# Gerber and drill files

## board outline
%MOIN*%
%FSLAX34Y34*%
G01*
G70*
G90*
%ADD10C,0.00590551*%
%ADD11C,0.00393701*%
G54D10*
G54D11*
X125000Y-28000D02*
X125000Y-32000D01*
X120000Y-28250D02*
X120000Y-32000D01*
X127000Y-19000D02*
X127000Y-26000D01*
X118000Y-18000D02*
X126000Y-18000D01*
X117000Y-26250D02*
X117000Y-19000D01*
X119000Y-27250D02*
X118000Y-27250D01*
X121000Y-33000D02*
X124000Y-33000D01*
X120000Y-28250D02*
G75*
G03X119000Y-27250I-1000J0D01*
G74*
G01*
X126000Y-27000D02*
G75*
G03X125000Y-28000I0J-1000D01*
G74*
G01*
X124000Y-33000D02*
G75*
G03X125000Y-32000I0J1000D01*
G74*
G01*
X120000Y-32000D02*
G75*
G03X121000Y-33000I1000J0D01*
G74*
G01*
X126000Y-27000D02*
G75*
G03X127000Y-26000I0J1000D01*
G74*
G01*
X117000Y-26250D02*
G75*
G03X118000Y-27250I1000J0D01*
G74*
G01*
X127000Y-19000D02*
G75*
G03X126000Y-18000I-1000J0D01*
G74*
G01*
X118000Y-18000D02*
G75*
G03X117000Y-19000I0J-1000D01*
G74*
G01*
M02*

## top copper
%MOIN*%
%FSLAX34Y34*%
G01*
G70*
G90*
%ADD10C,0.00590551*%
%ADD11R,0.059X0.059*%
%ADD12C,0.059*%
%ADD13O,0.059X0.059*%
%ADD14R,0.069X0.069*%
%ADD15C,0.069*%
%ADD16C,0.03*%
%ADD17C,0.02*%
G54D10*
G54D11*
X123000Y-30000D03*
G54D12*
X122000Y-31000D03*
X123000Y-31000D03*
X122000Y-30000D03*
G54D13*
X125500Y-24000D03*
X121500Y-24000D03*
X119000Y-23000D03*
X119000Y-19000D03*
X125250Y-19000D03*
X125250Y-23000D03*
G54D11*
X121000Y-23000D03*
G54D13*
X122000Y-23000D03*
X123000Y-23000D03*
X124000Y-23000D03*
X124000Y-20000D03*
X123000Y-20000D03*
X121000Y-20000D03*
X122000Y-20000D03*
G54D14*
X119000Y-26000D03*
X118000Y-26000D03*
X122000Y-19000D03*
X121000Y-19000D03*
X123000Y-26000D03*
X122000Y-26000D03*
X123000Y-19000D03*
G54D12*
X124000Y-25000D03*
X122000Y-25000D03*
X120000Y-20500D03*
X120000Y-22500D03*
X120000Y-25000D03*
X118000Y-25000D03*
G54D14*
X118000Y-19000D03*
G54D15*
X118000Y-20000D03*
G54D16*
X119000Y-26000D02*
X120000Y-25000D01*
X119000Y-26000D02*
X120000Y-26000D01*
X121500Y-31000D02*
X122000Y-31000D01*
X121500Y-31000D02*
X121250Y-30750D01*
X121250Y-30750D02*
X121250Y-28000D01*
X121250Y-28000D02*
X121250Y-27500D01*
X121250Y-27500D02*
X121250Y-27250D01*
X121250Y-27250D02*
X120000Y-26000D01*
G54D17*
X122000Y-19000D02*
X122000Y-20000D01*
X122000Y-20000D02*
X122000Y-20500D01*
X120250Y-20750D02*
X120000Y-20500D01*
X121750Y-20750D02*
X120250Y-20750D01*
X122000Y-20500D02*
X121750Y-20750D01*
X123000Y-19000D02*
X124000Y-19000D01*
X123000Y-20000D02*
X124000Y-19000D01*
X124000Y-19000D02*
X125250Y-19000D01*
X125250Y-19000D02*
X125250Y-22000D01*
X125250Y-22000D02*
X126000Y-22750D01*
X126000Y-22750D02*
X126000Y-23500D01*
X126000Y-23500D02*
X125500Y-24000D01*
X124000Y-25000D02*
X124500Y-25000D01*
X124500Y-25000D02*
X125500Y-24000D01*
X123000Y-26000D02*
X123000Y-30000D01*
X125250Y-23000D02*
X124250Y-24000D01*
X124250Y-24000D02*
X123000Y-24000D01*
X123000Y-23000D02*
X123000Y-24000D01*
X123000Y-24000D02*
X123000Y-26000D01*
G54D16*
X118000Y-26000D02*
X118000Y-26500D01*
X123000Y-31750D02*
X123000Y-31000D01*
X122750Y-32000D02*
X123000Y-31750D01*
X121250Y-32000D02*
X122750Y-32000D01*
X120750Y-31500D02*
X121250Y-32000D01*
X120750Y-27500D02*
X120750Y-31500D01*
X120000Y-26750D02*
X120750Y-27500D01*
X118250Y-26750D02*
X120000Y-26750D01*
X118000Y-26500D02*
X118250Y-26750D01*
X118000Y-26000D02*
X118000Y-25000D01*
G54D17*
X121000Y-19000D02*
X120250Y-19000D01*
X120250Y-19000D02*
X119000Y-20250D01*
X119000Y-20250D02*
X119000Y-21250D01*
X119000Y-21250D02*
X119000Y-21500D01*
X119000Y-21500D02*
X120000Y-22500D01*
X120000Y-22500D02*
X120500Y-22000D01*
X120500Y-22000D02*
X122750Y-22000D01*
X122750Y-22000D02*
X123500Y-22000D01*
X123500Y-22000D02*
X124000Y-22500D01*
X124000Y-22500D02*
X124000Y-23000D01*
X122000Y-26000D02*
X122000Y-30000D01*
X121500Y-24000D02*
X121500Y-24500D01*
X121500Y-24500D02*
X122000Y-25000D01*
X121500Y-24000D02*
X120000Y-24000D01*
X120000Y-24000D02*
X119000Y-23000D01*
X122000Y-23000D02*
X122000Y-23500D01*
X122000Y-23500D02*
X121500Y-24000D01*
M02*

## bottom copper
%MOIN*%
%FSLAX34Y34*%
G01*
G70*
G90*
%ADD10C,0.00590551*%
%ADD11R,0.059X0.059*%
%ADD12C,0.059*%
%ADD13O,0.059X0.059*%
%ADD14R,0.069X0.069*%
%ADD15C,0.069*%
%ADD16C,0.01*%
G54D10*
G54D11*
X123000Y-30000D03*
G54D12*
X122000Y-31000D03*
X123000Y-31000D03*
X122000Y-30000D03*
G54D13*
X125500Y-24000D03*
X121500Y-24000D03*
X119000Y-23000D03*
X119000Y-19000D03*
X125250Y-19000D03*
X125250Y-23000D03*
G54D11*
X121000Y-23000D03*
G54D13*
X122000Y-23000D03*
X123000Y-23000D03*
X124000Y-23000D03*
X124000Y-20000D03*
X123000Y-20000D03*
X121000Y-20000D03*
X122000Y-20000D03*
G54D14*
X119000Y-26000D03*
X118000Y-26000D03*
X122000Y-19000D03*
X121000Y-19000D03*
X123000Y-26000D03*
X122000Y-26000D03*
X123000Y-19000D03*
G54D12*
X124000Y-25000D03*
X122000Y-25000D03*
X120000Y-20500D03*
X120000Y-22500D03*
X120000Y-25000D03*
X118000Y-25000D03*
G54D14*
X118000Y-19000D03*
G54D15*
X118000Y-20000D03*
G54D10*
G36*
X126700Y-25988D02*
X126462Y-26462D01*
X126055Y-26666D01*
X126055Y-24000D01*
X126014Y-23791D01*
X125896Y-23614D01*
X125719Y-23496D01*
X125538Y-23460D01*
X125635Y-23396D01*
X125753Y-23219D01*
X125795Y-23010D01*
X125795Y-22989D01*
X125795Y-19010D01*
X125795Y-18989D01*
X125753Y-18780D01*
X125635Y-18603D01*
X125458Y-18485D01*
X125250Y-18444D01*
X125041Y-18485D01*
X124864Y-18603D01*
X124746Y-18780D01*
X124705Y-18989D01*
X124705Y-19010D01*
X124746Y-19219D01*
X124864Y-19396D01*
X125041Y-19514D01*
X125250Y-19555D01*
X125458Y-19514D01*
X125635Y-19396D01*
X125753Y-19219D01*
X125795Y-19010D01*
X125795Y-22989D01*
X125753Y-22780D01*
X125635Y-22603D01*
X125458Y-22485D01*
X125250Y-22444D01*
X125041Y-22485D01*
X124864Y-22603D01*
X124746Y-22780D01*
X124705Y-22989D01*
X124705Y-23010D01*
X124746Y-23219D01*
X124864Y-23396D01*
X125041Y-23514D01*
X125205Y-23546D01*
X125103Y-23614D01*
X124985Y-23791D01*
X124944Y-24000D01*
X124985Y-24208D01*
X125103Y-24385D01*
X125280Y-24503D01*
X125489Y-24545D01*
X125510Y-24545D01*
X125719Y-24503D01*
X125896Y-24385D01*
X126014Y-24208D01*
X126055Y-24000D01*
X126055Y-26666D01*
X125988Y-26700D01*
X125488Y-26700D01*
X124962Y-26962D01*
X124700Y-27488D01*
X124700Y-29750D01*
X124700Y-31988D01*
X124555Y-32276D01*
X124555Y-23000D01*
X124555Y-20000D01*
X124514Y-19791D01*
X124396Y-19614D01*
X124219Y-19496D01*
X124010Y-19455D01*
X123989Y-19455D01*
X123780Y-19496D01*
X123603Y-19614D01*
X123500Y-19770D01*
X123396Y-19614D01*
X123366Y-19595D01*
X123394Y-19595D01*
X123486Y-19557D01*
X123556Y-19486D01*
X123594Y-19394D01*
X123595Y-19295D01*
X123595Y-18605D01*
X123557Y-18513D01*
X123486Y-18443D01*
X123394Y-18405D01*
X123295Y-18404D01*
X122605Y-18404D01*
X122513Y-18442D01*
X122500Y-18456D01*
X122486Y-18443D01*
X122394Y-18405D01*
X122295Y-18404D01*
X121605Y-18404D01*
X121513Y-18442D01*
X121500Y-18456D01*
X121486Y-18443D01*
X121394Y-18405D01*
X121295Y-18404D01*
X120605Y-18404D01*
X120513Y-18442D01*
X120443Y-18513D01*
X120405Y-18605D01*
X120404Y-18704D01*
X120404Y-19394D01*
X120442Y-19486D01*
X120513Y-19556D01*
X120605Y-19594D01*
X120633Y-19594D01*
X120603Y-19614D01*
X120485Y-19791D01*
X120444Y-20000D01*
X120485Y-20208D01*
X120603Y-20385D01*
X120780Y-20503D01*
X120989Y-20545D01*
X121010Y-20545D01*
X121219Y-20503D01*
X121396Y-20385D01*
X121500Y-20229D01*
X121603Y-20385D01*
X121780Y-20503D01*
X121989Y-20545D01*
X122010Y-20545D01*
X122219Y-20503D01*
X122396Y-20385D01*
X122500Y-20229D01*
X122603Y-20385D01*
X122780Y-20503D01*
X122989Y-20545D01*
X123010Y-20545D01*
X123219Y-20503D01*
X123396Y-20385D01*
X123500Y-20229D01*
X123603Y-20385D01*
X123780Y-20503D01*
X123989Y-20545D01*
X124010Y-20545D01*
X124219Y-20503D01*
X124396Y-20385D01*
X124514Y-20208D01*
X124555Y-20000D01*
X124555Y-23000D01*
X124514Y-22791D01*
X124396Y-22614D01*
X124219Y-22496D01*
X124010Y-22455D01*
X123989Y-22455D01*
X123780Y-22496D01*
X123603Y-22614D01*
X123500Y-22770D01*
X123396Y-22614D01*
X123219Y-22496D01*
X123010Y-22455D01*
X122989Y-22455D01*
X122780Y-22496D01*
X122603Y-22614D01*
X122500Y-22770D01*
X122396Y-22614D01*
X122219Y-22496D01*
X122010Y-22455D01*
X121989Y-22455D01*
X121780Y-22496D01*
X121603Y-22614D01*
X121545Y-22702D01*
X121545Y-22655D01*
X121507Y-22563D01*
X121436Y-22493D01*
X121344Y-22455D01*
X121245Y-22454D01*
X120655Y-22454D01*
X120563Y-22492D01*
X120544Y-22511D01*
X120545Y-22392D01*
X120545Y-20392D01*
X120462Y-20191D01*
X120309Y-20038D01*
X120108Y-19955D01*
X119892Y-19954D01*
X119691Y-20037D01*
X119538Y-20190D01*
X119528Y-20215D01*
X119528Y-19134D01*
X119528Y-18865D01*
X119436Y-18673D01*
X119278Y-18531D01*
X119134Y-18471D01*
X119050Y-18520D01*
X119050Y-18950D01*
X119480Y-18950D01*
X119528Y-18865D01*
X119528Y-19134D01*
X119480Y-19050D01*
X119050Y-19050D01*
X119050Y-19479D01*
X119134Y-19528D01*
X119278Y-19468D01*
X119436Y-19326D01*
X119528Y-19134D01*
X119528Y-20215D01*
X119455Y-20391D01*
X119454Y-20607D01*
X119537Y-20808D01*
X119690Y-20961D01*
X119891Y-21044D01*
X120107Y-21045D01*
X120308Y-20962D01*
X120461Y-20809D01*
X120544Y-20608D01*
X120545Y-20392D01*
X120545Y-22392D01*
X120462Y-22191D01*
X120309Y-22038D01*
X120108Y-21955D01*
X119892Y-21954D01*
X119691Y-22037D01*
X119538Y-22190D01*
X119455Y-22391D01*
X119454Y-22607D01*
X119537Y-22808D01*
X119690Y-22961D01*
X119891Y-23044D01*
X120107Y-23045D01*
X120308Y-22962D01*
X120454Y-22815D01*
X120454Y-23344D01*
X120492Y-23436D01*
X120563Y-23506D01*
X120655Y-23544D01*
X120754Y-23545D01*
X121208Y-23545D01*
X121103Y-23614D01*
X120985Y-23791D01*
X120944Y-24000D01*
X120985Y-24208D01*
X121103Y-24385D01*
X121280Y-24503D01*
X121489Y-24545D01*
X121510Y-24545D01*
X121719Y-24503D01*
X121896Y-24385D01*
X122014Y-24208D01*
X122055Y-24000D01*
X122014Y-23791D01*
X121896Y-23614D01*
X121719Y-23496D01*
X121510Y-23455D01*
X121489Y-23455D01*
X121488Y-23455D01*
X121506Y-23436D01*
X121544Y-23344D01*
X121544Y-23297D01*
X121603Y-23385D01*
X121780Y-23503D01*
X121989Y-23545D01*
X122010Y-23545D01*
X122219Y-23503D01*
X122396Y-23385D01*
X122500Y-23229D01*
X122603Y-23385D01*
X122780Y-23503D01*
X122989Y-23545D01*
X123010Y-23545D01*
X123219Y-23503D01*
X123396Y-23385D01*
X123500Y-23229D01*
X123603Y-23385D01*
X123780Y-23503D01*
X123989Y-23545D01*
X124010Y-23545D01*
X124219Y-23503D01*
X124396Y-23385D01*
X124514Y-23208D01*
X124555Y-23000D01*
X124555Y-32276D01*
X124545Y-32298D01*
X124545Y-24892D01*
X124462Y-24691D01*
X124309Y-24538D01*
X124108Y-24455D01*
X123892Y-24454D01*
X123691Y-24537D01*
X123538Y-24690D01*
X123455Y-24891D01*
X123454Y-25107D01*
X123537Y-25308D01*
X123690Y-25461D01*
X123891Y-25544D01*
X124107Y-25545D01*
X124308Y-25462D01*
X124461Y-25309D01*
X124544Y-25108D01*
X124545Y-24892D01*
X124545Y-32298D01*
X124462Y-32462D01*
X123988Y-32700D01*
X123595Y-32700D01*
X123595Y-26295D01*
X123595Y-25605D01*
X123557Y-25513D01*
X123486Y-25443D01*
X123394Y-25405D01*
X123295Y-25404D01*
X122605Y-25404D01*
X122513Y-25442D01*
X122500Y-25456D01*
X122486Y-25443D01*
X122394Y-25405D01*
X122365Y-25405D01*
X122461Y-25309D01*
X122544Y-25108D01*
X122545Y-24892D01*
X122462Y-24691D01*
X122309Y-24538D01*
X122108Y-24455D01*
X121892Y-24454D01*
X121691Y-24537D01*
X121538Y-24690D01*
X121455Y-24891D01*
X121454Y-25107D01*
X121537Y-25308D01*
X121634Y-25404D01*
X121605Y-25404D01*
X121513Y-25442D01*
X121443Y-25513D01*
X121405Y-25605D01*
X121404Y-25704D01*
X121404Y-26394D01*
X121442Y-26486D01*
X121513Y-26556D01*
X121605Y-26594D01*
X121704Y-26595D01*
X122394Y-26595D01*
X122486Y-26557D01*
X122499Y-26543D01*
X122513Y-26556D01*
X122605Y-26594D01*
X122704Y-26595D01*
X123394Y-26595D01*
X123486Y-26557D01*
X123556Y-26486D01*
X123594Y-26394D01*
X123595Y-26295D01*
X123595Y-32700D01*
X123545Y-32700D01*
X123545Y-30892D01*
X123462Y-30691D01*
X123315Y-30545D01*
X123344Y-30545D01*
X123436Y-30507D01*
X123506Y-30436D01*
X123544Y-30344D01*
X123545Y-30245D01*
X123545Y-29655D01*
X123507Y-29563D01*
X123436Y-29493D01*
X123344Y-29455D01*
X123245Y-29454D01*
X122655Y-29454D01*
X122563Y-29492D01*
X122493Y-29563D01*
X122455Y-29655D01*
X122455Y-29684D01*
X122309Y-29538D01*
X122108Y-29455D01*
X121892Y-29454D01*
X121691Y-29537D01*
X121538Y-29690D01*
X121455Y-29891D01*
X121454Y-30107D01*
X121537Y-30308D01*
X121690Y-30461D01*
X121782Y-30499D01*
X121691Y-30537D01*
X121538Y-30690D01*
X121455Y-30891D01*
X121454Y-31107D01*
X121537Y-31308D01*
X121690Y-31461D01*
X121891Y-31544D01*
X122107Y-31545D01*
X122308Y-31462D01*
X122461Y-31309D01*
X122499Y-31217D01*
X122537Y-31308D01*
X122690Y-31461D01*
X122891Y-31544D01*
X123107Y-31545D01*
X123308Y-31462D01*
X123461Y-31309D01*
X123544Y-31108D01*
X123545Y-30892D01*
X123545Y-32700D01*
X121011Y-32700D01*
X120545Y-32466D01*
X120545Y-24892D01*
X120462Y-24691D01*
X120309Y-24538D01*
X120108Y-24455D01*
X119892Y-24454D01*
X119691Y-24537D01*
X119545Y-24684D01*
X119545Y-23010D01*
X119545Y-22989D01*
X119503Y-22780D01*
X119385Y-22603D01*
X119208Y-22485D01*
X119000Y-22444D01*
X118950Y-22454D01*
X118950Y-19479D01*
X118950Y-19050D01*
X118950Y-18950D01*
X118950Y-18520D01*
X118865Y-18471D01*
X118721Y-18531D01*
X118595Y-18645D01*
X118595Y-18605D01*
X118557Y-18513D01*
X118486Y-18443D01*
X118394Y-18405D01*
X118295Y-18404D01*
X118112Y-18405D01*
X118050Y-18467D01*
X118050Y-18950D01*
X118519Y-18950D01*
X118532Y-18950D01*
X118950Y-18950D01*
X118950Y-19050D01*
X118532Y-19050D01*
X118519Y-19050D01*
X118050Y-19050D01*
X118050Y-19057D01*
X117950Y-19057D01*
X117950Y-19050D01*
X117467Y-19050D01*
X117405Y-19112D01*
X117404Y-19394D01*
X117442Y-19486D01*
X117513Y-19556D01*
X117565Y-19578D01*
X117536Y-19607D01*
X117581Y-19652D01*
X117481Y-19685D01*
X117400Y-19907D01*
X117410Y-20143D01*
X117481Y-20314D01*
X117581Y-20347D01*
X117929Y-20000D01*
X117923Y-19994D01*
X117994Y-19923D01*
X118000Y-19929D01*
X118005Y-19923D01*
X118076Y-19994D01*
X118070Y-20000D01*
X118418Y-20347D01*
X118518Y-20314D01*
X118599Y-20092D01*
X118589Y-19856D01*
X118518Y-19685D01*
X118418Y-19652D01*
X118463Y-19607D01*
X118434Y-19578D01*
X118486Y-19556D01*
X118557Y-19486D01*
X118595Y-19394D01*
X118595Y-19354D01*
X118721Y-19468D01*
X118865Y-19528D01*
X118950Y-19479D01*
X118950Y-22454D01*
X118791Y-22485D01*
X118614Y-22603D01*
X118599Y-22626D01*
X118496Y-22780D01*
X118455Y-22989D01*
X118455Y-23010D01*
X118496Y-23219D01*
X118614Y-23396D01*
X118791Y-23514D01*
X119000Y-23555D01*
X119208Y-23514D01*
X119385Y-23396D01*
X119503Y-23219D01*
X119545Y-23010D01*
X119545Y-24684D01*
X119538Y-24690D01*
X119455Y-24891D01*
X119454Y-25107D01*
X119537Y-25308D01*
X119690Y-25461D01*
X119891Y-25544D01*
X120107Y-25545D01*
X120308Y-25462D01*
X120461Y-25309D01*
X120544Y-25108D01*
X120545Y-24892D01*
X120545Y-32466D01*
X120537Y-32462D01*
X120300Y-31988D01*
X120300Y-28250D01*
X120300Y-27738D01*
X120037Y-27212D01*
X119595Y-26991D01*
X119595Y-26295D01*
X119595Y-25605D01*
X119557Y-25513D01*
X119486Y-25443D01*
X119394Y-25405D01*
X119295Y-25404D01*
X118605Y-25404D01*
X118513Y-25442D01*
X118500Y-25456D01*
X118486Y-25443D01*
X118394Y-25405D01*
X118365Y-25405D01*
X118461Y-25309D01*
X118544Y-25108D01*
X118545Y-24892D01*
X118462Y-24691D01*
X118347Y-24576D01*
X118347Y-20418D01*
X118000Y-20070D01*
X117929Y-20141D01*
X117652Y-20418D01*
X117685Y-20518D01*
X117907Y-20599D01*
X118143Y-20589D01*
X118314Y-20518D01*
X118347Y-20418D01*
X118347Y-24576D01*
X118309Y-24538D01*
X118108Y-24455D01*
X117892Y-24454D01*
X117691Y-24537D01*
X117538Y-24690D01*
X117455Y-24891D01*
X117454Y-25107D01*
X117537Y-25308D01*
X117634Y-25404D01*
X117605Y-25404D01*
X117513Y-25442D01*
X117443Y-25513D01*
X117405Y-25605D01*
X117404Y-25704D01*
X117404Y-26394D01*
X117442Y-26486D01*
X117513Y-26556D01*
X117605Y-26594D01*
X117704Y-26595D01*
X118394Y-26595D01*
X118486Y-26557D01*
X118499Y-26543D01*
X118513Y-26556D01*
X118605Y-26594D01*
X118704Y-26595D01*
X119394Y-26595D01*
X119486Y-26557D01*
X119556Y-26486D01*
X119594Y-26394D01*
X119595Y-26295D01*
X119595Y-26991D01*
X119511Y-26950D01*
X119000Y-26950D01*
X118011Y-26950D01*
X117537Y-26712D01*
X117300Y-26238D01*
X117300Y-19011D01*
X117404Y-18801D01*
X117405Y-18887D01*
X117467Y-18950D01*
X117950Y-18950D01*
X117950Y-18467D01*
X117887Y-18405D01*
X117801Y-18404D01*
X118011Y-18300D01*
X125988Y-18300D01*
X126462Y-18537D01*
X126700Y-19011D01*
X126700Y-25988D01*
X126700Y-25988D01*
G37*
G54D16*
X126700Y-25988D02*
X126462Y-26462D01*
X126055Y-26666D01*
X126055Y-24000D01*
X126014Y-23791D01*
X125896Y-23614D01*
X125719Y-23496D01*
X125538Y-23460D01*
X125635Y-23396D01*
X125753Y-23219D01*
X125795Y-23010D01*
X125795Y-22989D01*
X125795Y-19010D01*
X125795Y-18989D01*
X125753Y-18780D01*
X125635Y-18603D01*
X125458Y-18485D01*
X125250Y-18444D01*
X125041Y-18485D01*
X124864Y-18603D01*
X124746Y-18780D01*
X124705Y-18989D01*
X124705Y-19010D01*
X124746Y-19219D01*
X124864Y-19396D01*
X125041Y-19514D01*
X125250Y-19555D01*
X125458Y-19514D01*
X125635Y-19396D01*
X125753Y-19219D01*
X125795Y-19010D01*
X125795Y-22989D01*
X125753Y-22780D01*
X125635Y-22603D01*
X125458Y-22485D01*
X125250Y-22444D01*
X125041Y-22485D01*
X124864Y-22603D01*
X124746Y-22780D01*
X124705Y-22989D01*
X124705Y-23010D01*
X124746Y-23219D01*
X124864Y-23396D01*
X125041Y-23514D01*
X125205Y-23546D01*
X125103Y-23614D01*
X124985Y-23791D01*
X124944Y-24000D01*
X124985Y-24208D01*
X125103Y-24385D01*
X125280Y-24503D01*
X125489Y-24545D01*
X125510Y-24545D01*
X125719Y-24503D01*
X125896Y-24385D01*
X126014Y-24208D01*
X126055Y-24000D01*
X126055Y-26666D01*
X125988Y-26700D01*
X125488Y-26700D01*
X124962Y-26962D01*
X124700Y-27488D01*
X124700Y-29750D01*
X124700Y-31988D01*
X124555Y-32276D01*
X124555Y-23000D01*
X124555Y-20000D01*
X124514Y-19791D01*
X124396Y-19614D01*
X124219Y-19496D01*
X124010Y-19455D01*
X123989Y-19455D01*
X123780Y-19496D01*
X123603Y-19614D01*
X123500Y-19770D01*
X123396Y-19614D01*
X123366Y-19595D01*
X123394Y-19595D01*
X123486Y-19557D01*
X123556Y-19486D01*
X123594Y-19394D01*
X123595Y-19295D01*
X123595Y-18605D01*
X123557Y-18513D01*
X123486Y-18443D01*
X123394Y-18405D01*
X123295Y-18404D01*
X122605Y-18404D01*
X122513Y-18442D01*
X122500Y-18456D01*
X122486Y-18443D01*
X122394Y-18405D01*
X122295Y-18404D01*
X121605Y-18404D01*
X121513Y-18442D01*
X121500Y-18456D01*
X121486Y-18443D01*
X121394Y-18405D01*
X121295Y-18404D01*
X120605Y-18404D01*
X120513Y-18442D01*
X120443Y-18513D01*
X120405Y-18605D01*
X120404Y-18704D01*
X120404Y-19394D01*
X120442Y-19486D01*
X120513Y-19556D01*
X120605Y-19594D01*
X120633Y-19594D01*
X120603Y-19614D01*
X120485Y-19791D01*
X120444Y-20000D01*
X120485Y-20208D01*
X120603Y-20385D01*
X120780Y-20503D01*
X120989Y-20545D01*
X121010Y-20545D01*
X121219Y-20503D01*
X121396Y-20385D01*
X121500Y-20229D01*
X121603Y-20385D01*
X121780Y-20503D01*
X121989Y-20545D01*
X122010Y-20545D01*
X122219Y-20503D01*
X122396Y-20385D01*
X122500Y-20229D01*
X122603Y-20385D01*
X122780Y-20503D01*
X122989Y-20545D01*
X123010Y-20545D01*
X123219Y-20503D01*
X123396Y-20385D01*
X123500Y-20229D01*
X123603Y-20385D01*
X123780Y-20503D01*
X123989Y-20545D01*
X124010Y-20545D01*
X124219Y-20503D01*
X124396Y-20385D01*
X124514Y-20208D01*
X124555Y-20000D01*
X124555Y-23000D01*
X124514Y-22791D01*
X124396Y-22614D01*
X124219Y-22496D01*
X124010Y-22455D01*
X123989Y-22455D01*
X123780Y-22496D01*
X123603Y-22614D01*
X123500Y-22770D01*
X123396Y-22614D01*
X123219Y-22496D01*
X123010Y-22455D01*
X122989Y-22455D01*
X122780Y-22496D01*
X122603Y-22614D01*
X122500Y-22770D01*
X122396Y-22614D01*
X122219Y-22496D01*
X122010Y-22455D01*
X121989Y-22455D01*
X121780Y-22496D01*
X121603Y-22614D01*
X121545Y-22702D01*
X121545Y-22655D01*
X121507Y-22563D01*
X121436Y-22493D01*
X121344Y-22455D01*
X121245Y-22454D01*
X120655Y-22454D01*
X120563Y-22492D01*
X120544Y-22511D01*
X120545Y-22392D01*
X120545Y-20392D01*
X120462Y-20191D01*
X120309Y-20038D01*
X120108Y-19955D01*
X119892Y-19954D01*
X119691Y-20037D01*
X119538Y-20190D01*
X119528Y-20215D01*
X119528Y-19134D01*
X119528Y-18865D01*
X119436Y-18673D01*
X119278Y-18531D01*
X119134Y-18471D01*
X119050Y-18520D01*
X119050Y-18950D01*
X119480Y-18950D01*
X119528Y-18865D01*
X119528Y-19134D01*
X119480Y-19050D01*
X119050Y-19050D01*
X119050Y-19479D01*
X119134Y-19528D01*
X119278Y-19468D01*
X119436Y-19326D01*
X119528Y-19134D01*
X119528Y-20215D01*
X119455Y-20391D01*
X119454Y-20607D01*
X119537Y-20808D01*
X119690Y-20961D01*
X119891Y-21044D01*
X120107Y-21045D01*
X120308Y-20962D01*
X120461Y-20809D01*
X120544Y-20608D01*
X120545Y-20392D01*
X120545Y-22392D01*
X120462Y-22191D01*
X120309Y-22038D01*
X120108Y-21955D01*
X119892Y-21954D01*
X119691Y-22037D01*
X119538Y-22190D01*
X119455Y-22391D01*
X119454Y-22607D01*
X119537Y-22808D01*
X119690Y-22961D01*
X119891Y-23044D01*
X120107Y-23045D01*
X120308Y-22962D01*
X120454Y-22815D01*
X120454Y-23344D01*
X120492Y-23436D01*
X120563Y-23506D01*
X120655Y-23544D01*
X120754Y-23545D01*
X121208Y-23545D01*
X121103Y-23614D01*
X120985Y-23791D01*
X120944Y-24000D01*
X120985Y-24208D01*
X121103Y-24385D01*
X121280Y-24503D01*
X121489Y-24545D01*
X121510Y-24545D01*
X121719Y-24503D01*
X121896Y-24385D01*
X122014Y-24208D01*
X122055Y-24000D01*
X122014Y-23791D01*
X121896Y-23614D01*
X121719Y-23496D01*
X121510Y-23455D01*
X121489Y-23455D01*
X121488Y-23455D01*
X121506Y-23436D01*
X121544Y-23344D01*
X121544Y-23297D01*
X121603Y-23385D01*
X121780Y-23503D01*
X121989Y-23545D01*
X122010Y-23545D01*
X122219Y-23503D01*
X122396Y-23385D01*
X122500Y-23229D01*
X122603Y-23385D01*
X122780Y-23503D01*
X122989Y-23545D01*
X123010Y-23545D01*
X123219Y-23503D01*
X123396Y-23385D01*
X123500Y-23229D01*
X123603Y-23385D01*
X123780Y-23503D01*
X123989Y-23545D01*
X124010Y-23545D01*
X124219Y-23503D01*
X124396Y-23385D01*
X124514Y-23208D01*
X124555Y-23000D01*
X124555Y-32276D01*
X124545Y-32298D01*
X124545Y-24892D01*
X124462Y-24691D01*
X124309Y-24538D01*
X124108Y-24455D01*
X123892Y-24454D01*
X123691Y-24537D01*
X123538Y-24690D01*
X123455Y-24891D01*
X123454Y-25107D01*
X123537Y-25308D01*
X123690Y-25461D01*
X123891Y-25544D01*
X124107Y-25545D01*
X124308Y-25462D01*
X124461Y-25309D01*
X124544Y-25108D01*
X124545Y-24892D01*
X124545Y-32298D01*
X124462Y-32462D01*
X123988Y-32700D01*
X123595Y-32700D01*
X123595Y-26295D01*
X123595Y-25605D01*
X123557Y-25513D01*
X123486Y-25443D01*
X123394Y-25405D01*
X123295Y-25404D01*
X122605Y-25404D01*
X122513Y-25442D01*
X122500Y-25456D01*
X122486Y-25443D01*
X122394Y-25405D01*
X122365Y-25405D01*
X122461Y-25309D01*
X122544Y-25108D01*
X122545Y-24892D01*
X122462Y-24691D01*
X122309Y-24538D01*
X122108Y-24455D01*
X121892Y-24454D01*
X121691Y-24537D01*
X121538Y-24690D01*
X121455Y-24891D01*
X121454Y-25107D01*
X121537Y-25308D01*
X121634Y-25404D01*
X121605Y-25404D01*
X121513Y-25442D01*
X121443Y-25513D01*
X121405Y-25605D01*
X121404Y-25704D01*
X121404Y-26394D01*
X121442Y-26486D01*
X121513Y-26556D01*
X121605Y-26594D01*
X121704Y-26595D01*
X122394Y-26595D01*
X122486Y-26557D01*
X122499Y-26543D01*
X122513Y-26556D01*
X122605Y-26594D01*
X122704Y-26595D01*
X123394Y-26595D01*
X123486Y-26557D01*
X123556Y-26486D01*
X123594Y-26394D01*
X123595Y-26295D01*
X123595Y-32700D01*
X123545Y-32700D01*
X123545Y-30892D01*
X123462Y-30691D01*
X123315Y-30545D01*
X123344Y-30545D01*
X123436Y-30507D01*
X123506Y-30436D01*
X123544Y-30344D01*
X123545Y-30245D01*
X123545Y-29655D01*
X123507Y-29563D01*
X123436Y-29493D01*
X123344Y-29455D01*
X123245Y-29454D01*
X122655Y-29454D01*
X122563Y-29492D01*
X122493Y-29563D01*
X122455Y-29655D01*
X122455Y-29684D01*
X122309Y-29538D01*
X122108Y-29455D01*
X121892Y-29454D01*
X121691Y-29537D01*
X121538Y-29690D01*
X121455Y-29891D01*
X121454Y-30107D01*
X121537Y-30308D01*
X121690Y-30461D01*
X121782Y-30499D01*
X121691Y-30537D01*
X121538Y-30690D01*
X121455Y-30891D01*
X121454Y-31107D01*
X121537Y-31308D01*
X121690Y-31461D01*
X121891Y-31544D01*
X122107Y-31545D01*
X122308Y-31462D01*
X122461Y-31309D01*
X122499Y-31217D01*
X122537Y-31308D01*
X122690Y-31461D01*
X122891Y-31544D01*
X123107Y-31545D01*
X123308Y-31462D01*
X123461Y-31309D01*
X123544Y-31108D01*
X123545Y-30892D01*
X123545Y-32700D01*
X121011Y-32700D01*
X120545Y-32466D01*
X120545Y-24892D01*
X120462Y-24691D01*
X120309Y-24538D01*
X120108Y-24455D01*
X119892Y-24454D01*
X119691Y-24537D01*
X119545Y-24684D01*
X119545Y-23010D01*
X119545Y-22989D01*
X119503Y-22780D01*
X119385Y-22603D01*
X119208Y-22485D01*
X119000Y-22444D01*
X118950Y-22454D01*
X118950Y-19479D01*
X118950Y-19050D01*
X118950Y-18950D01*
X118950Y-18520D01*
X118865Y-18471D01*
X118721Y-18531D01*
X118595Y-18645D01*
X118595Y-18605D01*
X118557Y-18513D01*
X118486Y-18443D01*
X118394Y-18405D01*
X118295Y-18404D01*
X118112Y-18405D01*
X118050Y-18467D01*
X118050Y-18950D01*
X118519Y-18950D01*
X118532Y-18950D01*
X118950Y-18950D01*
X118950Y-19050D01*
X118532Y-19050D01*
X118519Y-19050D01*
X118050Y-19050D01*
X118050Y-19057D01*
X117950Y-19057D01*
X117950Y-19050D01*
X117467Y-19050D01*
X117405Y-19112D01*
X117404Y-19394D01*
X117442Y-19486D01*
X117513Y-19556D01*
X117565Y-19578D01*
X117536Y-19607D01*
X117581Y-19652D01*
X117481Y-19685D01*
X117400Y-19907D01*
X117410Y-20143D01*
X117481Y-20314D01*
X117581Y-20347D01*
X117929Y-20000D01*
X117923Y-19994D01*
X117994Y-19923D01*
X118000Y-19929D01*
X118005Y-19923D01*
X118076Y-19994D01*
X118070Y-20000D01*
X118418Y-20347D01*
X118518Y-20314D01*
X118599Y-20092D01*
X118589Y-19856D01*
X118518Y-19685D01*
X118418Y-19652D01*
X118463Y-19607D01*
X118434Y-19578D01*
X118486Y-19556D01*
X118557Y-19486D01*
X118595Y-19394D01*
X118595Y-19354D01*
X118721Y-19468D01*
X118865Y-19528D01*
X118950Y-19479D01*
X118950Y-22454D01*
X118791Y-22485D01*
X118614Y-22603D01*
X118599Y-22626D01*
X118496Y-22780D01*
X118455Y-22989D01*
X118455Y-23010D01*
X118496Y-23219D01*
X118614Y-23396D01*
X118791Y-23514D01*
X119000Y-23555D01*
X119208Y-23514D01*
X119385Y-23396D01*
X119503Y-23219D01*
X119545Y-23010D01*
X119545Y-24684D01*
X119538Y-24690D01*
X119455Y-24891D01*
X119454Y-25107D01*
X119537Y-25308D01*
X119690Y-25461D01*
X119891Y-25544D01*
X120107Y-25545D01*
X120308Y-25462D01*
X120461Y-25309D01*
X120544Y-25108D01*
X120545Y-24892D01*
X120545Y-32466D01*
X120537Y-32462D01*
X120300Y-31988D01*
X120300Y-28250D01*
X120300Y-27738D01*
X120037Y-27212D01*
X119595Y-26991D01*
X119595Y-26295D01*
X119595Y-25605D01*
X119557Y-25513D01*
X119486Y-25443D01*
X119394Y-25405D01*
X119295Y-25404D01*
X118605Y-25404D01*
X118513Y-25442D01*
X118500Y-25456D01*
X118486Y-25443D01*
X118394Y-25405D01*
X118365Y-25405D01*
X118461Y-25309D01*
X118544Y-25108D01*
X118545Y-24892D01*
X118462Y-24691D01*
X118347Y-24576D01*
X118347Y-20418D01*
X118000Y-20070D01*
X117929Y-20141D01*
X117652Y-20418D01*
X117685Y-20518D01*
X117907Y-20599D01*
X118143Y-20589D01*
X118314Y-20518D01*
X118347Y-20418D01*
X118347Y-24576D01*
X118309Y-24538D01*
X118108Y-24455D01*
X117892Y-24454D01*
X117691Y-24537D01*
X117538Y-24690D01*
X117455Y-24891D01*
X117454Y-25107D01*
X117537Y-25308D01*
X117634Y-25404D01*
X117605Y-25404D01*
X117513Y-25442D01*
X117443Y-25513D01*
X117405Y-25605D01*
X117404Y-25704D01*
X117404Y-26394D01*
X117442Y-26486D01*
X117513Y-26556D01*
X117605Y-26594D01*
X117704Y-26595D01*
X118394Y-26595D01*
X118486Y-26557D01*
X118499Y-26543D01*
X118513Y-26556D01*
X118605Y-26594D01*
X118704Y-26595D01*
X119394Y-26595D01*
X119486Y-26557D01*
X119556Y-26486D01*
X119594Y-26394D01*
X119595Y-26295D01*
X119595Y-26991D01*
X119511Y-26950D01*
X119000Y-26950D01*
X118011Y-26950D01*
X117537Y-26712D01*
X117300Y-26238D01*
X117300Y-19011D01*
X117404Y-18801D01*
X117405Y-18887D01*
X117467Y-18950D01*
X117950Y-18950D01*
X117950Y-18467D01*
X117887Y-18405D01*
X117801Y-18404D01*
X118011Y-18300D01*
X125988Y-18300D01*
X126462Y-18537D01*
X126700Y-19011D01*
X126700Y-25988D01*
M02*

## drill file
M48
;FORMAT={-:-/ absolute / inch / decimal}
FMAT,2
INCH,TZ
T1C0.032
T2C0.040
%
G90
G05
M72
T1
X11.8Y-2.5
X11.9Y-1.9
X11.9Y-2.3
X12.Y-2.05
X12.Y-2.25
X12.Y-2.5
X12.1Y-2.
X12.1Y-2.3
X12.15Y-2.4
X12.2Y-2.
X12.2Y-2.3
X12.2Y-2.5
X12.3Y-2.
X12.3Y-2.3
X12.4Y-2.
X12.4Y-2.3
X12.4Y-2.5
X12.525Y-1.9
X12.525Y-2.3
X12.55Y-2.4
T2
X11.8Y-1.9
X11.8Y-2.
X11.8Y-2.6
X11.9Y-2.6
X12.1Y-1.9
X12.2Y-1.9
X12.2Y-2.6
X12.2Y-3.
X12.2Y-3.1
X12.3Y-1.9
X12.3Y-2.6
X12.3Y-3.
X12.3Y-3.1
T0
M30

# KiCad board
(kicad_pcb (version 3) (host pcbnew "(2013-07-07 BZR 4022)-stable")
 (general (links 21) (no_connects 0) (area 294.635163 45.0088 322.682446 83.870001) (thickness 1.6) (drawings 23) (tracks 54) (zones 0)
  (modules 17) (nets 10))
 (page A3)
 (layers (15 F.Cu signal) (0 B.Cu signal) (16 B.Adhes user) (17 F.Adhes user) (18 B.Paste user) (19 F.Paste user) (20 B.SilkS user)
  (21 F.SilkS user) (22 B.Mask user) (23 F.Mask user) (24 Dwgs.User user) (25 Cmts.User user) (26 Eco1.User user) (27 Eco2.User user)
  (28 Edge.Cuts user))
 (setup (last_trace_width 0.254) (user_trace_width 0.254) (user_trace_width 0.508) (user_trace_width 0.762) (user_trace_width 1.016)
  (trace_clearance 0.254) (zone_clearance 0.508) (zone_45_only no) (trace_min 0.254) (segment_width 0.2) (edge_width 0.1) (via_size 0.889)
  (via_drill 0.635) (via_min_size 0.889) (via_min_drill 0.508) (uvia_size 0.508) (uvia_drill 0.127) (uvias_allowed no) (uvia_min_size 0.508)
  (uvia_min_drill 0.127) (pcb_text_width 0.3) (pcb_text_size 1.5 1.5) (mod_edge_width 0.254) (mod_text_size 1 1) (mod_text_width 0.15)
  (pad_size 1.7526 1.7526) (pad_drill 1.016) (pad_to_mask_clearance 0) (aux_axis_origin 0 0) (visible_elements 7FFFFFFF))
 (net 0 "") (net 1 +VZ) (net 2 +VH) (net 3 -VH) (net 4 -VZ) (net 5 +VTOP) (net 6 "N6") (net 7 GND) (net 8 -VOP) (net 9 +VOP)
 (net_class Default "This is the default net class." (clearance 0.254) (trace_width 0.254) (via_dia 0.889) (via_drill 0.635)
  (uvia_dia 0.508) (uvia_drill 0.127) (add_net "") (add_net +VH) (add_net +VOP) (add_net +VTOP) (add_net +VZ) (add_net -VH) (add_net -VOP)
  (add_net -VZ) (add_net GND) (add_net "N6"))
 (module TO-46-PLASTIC (layer F.Cu) (at 311.15 77.47 270)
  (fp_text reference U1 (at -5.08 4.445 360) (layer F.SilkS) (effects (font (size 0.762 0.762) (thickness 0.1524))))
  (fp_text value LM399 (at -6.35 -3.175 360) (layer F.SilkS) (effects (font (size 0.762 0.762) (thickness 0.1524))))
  (pad 1 thru_hole rect (at -1.27 -1.27 270) (size 1.4986 1.4986) (drill 1.016) (layers *.Cu *.Mask F.SilkS) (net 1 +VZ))
  (pad 3 thru_hole circle (at 1.27 1.27 270) (size 1.4986 1.4986) (drill 1.016) (layers *.Cu *.Mask F.SilkS) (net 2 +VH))
  (pad 4 thru_hole circle (at 1.27 -1.27 270) (size 1.4986 1.4986) (drill 1.016) (layers *.Cu *.Mask F.SilkS) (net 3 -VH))
  (pad 2 thru_hole circle (at -1.27 1.27 270) (size 1.4986 1.4986) (drill 1.016) (layers *.Cu *.Mask F.SilkS) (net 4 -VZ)))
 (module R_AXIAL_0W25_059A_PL (layer F.Cu) (at 318.77 60.96 180) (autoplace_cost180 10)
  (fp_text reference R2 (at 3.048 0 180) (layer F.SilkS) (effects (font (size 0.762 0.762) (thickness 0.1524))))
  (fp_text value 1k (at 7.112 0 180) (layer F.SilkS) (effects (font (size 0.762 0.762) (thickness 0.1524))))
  (pad 1 thru_hole oval (at 0 0 180) (size 1.4986 1.4986) (drill 0.8128) (layers *.Cu *.Mask F.SilkS) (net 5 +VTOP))
  (pad 2 thru_hole oval (at 10.16 0 180) (size 1.4986 1.4986) (drill 0.8128) (layers *.Cu *.Mask F.SilkS) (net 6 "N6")))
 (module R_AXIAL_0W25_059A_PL (layer F.Cu) (at 302.26 58.42 90) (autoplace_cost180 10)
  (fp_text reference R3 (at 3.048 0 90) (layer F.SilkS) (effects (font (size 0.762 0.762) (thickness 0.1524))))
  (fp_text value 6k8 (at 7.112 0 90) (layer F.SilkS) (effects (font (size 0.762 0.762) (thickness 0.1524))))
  (pad 1 thru_hole oval (at 0 0 90) (size 1.4986 1.4986) (drill 0.8128) (layers *.Cu *.Mask F.SilkS) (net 6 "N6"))
  (pad 2 thru_hole oval (at 10.16 0 90) (size 1.4986 1.4986) (drill 0.8128) (layers *.Cu *.Mask F.SilkS) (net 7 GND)))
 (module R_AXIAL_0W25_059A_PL (layer F.Cu) (at 318.135 48.26 270) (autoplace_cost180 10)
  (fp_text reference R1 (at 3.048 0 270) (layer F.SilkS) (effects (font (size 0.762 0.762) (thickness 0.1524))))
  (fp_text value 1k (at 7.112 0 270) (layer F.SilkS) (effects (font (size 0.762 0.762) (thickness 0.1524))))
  (pad 1 thru_hole oval (at 0 0 270) (size 1.4986 1.4986) (drill 0.8128) (layers *.Cu *.Mask F.SilkS) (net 5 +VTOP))
  (pad 2 thru_hole oval (at 10.16 0 270) (size 1.4986 1.4986) (drill 0.8128) (layers *.Cu *.Mask F.SilkS) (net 1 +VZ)))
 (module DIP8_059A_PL (layer F.Cu) (at 307.34 58.42)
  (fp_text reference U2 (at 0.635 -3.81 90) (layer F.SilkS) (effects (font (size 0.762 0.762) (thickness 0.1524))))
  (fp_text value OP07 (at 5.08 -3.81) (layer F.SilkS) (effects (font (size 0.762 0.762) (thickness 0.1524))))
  (pad 1 thru_hole rect (at 0 0) (size 1.4986 1.4986) (drill 0.8128) (layers *.Cu *.Mask F.SilkS))
  (pad 2 thru_hole oval (at 2.54 0) (size 1.4986 1.4986) (drill 0.8128) (layers *.Cu *.Mask F.SilkS) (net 6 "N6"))
  (pad 3 thru_hole oval (at 5.08 0) (size 1.4986 1.4986) (drill 0.8128) (layers *.Cu *.Mask F.SilkS) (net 1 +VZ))
  (pad 4 thru_hole oval (at 7.62 0) (size 1.4986 1.4986) (drill 0.8128) (layers *.Cu *.Mask F.SilkS) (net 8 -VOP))
  (pad 5 thru_hole oval (at 7.62 -7.62) (size 1.4986 1.4986) (drill 0.8128) (layers *.Cu *.Mask F.SilkS))
  (pad 6 thru_hole oval (at 5.08 -7.62) (size 1.4986 1.4986) (drill 0.8128) (layers *.Cu *.Mask F.SilkS) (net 5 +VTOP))
  (pad 8 thru_hole oval (at 0 -7.62) (size 1.4986 1.4986) (drill 0.8128) (layers *.Cu *.Mask F.SilkS))
  (pad 7 thru_hole oval (at 2.54 -7.62) (size 1.4986 1.4986) (drill 0.8128) (layers *.Cu *.Mask F.SilkS) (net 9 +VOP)))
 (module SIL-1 (layer F.Cu) (at 302.26 66.04)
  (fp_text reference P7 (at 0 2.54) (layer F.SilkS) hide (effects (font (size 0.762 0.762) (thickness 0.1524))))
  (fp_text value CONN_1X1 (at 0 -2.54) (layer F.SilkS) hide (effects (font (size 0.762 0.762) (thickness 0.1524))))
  (pad 1 thru_hole rect (at 0 0) (size 1.7526 1.7526) (drill 1.016) (layers *.Cu *.Mask F.SilkS) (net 2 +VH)))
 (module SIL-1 (layer F.Cu) (at 299.72 66.04)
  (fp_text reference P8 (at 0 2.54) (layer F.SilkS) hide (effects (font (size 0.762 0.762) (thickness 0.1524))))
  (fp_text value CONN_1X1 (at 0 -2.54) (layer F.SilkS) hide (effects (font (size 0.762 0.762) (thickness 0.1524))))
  (pad 1 thru_hole rect (at 0 0) (size 1.7526 1.7526) (drill 1.016) (layers *.Cu *.Mask F.SilkS) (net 3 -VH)))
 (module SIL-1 (layer F.Cu) (at 309.88 48.26)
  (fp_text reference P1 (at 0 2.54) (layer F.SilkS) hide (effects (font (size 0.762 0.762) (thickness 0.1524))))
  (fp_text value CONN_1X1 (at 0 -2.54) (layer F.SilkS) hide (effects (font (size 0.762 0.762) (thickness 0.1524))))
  (pad 1 thru_hole rect (at 0 0) (size 1.7526 1.7526) (drill 1.016) (layers *.Cu *.Mask F.SilkS) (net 9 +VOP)))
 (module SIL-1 (layer F.Cu) (at 307.34 48.26)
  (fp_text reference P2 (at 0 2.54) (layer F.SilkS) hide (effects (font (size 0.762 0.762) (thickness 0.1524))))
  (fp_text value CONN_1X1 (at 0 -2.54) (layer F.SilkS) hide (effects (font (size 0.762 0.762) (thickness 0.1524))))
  (pad 1 thru_hole rect (at 0 0) (size 1.7526 1.7526) (drill 1.016) (layers *.Cu *.Mask F.SilkS) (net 8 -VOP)))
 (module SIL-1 (layer F.Cu) (at 312.42 66.04)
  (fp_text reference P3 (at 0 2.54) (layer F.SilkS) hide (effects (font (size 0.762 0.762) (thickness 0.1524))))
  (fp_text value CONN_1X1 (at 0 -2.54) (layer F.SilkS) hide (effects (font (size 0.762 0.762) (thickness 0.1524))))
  (pad 1 thru_hole rect (at 0 0) (size 1.7526 1.7526) (drill 1.016) (layers *.Cu *.Mask F.SilkS) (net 1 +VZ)))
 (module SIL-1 (layer F.Cu) (at 309.88 66.04)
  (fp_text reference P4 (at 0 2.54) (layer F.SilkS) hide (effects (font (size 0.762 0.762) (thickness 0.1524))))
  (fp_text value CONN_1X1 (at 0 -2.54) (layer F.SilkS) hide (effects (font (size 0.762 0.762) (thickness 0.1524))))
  (pad 1 thru_hole rect (at 0 0) (size 1.7526 1.7526) (drill 1.016) (layers *.Cu *.Mask F.SilkS) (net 4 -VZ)))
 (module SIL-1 (layer F.Cu) (at 312.42 48.26)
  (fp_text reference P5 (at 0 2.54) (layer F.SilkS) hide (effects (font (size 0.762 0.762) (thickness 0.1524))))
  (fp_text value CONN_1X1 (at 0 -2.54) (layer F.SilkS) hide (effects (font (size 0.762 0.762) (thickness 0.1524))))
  (pad 1 thru_hole rect (at 0 0) (size 1.7526 1.7526) (drill 1.016) (layers *.Cu *.Mask F.SilkS) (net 5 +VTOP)))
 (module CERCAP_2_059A (layer F.Cu) (at 312.42 63.5 180)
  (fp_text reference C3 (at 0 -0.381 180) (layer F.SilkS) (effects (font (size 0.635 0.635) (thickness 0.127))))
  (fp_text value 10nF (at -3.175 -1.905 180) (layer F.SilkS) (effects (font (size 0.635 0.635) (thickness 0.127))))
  (pad 1 thru_hole circle (at -2.54 0 180) (size 1.4986 1.4986) (drill 0.8128) (layers *.Cu *.Mask F.SilkS) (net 5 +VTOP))
  (pad 2 thru_hole circle (at 2.54 0 180) (size 1.4986 1.4986) (drill 0.8128) (layers *.Cu *.Mask F.SilkS) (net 6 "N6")))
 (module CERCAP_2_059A (layer F.Cu) (at 304.8 54.61 270)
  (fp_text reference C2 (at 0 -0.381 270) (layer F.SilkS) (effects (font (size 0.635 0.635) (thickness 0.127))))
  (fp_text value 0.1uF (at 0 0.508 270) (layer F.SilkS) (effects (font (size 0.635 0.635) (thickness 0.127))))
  (pad 1 thru_hole circle (at -2.54 0 270) (size 1.4986 1.4986) (drill 0.8128) (layers *.Cu *.Mask F.SilkS) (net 9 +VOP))
  (pad 2 thru_hole circle (at 2.54 0 270) (size 1.4986 1.4986) (drill 0.8128) (layers *.Cu *.Mask F.SilkS) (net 8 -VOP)))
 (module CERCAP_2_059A (layer F.Cu) (at 302.26 63.5 180)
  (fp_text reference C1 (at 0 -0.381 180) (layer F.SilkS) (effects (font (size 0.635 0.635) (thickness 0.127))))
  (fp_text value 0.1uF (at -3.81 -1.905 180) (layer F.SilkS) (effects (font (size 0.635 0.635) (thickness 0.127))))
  (pad 1 thru_hole circle (at -2.54 0 180) (size 1.4986 1.4986) (drill 0.8128) (layers *.Cu *.Mask F.SilkS) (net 2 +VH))
  (pad 2 thru_hole circle (at 2.54 0 180) (size 1.4986 1.4986) (drill 0.8128) (layers *.Cu *.Mask F.SilkS) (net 3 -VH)))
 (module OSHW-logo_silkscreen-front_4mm (layer F.Cu) (at 319.405 65.405)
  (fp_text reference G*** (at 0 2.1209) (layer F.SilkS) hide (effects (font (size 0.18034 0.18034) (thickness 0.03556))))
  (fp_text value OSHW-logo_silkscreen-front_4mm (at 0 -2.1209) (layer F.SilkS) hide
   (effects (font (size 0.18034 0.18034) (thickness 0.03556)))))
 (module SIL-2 (layer F.Cu) (at 299.72 48.26 270)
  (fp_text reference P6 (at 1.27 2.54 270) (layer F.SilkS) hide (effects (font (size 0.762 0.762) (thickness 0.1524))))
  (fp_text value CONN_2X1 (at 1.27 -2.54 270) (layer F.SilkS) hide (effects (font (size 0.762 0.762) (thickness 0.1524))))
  (pad 1 thru_hole rect (at 0 0 270) (size 1.7526 1.7526) (drill 1.016) (layers *.Cu *.Mask F.SilkS) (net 7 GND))
  (pad 2 thru_hole circle (at 2.54 0 270) (size 1.7526 1.7526) (drill 1.016) (layers *.Cu *.Mask F.SilkS) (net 7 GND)))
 (gr_line (start 317.5 71.12) (end 317.5 81.28) (angle 90) (layer Edge.Cuts) (width 0.1))
 (gr_line (start 304.8 71.755) (end 304.8 81.28) (angle 90) (layer Edge.Cuts) (width 0.1))
 (gr_line (start 322.58 48.26) (end 322.58 66.04) (angle 90) (layer Edge.Cuts) (width 0.1))
 (gr_line (start 299.72 45.72) (end 320.04 45.72) (angle 90) (layer Edge.Cuts) (width 0.1))
 (gr_line (start 297.18 66.675) (end 297.18 48.26) (angle 90) (layer Edge.Cuts) (width 0.1))
 (gr_line (start 302.26 69.215) (end 299.72 69.215) (angle 90) (layer Edge.Cuts) (width 0.1))
 (gr_line (start 307.34 83.82) (end 314.96 83.82) (angle 90) (layer Edge.Cuts) (width 0.1))
 (gr_arc (start 302.26 71.755) (end 302.26 69.215) (angle 90) (layer Edge.Cuts) (width 0.1))
 (gr_arc (start 320.04 71.12) (end 317.5 71.12) (angle 90) (layer Edge.Cuts) (width 0.1))
 (gr_arc (start 314.96 81.28) (end 317.5 81.28) (angle 90) (layer Edge.Cuts) (width 0.1))
 (gr_arc (start 307.34 81.28) (end 307.34 83.82) (angle 90) (layer Edge.Cuts) (width 0.1))
 (gr_arc (start 320.04 66.04) (end 322.58 66.04) (angle 90) (layer Edge.Cuts) (width 0.1))
 (gr_arc (start 299.72 66.675) (end 299.72 69.215) (angle 90) (layer Edge.Cuts) (width 0.1))
 (gr_arc (start 320.04 48.26) (end 320.04 45.72) (angle 90) (layer Edge.Cuts) (width 0.1))
 (gr_arc (start 299.72 48.26) (end 297.18 48.26) (angle 90) (layer Edge.Cuts) (width 0.1))
 (segment (start 302.26 66.04) (end 304.8 63.5) (width 0.762) (layer F.Cu) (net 2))
 (segment (start 302.26 66.04) (end 304.8 66.04) (width 0.762) (layer F.Cu) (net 2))
 (segment (start 308.61 78.74) (end 309.88 78.74) (width 0.762) (layer F.Cu) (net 2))
 (segment (start 308.61 78.74) (end 307.975 78.105) (width 0.762) (layer F.Cu) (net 2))
 (segment (start 307.975 78.105) (end 307.975 71.12) (width 0.762) (layer F.Cu) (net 2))
 (segment (start 307.975 71.12) (end 307.975 69.85) (width 0.762) (layer F.Cu) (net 2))
 (segment (start 307.975 69.85) (end 307.975 69.215) (width 0.762) (layer F.Cu) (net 2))
 (segment (start 307.975 69.215) (end 304.8 66.04) (width 0.762) (layer F.Cu) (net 2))
 (segment (start 309.88 48.26) (end 309.88 50.8) (width 0.508) (layer F.Cu) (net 9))
 (segment (start 309.88 50.8) (end 309.88 52.07) (width 0.508) (layer F.Cu) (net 9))
 (segment (start 305.435 52.705) (end 304.8 52.07) (width 0.508) (layer F.Cu) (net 9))
 (segment (start 309.245 52.705) (end 305.435 52.705) (width 0.508) (layer F.Cu) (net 9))
 (segment (start 309.88 52.07) (end 309.245 52.705) (width 0.508) (layer F.Cu) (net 9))
 (segment (start 312.42 48.26) (end 314.96 48.26) (width 0.508) (layer F.Cu) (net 5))
 (segment (start 312.42 50.8) (end 314.96 48.26) (width 0.508) (layer F.Cu) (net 5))
 (segment (start 314.96 48.26) (end 318.135 48.26) (width 0.508) (layer F.Cu) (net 5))
 (segment (start 318.135 48.26) (end 318.135 55.88) (width 0.508) (layer F.Cu) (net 5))
 (segment (start 318.135 55.88) (end 320.04 57.785) (width 0.508) (layer F.Cu) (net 5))
 (segment (start 320.04 57.785) (end 320.04 59.69) (width 0.508) (layer F.Cu) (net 5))
 (segment (start 320.04 59.69) (end 318.77 60.96) (width 0.508) (layer F.Cu) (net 5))
 (segment (start 314.96 63.5) (end 316.23 63.5) (width 0.508) (layer F.Cu) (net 5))
 (segment (start 316.23 63.5) (end 318.77 60.96) (width 0.508) (layer F.Cu) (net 5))
 (segment (start 312.42 66.04) (end 312.42 76.2) (width 0.508) (layer F.Cu) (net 1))
 (segment (start 318.135 58.42) (end 315.595 60.96) (width 0.508) (layer F.Cu) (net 1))
 (segment (start 315.595 60.96) (end 312.42 60.96) (width 0.508) (layer F.Cu) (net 1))
 (segment (start 312.42 58.42) (end 312.42 60.96) (width 0.508) (layer F.Cu) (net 1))
 (segment (start 312.42 60.96) (end 312.42 66.04) (width 0.508) (layer F.Cu) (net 1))
 (segment (start 299.72 66.04) (end 299.72 67.31) (width 0.762) (layer F.Cu) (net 3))
 (segment (start 312.42 80.645) (end 312.42 78.74) (width 0.762) (layer F.Cu) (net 3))
 (segment (start 311.785 81.28) (end 312.42 80.645) (width 0.762) (layer F.Cu) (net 3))
 (segment (start 307.975 81.28) (end 311.785 81.28) (width 0.762) (layer F.Cu) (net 3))
 (segment (start 306.705 80.01) (end 307.975 81.28) (width 0.762) (layer F.Cu) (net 3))
 (segment (start 306.705 69.85) (end 306.705 80.01) (width 0.762) (layer F.Cu) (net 3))
 (segment (start 304.8 67.945) (end 306.705 69.85) (width 0.762) (layer F.Cu) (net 3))
 (segment (start 300.355 67.945) (end 304.8 67.945) (width 0.762) (layer F.Cu) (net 3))
 (segment (start 299.72 67.31) (end 300.355 67.945) (width 0.762) (layer F.Cu) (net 3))
 (segment (start 299.72 66.04) (end 299.72 63.5) (width 0.762) (layer F.Cu) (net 3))
 (segment (start 307.34 48.26) (end 305.435 48.26) (width 0.508) (layer F.Cu) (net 8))
 (segment (start 305.435 48.26) (end 302.26 51.435) (width 0.508) (layer F.Cu) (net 8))
 (segment (start 302.26 51.435) (end 302.26 53.975) (width 0.508) (layer F.Cu) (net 8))
 (segment (start 302.26 53.975) (end 302.26 54.61) (width 0.508) (layer F.Cu) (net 8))
 (segment (start 302.26 54.61) (end 304.8 57.15) (width 0.508) (layer F.Cu) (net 8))
 (segment (start 304.8 57.15) (end 306.07 55.88) (width 0.508) (layer F.Cu) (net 8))
 (segment (start 306.07 55.88) (end 311.785 55.88) (width 0.508) (layer F.Cu) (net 8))
 (segment (start 311.785 55.88) (end 313.69 55.88) (width 0.508) (layer F.Cu) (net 8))
 (segment (start 313.69 55.88) (end 314.96 57.15) (width 0.508) (layer F.Cu) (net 8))
 (segment (start 314.96 57.15) (end 314.96 58.42) (width 0.508) (layer F.Cu) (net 8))
 (segment (start 309.88 66.04) (end 309.88 76.2) (width 0.508) (layer F.Cu) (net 4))
 (segment (start 308.61 60.96) (end 308.61 62.23) (width 0.508) (layer F.Cu) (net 6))
 (segment (start 308.61 62.23) (end 309.88 63.5) (width 0.508) (layer F.Cu) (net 6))
 (segment (start 308.61 60.96) (end 304.8 60.96) (width 0.508) (layer F.Cu) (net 6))
 (segment (start 304.8 60.96) (end 302.26 58.42) (width 0.508) (layer F.Cu) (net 6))
 (segment (start 309.88 58.42) (end 309.88 59.69) (width 0.508) (layer F.Cu) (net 6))
 (segment (start 309.88 59.69) (end 308.61 60.96) (width 0.508) (layer F.Cu) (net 6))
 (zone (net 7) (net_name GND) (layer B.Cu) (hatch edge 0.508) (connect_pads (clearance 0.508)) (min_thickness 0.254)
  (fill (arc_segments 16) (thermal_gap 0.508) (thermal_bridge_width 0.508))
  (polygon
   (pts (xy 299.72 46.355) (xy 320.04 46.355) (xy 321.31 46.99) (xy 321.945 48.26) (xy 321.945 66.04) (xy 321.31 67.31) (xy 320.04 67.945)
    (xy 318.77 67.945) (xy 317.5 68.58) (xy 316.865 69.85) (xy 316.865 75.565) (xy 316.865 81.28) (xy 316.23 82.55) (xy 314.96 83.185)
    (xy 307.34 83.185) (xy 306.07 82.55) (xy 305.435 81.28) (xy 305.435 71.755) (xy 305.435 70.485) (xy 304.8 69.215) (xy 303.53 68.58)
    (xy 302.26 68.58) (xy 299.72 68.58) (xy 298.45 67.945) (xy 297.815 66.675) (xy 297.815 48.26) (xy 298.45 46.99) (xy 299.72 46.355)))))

